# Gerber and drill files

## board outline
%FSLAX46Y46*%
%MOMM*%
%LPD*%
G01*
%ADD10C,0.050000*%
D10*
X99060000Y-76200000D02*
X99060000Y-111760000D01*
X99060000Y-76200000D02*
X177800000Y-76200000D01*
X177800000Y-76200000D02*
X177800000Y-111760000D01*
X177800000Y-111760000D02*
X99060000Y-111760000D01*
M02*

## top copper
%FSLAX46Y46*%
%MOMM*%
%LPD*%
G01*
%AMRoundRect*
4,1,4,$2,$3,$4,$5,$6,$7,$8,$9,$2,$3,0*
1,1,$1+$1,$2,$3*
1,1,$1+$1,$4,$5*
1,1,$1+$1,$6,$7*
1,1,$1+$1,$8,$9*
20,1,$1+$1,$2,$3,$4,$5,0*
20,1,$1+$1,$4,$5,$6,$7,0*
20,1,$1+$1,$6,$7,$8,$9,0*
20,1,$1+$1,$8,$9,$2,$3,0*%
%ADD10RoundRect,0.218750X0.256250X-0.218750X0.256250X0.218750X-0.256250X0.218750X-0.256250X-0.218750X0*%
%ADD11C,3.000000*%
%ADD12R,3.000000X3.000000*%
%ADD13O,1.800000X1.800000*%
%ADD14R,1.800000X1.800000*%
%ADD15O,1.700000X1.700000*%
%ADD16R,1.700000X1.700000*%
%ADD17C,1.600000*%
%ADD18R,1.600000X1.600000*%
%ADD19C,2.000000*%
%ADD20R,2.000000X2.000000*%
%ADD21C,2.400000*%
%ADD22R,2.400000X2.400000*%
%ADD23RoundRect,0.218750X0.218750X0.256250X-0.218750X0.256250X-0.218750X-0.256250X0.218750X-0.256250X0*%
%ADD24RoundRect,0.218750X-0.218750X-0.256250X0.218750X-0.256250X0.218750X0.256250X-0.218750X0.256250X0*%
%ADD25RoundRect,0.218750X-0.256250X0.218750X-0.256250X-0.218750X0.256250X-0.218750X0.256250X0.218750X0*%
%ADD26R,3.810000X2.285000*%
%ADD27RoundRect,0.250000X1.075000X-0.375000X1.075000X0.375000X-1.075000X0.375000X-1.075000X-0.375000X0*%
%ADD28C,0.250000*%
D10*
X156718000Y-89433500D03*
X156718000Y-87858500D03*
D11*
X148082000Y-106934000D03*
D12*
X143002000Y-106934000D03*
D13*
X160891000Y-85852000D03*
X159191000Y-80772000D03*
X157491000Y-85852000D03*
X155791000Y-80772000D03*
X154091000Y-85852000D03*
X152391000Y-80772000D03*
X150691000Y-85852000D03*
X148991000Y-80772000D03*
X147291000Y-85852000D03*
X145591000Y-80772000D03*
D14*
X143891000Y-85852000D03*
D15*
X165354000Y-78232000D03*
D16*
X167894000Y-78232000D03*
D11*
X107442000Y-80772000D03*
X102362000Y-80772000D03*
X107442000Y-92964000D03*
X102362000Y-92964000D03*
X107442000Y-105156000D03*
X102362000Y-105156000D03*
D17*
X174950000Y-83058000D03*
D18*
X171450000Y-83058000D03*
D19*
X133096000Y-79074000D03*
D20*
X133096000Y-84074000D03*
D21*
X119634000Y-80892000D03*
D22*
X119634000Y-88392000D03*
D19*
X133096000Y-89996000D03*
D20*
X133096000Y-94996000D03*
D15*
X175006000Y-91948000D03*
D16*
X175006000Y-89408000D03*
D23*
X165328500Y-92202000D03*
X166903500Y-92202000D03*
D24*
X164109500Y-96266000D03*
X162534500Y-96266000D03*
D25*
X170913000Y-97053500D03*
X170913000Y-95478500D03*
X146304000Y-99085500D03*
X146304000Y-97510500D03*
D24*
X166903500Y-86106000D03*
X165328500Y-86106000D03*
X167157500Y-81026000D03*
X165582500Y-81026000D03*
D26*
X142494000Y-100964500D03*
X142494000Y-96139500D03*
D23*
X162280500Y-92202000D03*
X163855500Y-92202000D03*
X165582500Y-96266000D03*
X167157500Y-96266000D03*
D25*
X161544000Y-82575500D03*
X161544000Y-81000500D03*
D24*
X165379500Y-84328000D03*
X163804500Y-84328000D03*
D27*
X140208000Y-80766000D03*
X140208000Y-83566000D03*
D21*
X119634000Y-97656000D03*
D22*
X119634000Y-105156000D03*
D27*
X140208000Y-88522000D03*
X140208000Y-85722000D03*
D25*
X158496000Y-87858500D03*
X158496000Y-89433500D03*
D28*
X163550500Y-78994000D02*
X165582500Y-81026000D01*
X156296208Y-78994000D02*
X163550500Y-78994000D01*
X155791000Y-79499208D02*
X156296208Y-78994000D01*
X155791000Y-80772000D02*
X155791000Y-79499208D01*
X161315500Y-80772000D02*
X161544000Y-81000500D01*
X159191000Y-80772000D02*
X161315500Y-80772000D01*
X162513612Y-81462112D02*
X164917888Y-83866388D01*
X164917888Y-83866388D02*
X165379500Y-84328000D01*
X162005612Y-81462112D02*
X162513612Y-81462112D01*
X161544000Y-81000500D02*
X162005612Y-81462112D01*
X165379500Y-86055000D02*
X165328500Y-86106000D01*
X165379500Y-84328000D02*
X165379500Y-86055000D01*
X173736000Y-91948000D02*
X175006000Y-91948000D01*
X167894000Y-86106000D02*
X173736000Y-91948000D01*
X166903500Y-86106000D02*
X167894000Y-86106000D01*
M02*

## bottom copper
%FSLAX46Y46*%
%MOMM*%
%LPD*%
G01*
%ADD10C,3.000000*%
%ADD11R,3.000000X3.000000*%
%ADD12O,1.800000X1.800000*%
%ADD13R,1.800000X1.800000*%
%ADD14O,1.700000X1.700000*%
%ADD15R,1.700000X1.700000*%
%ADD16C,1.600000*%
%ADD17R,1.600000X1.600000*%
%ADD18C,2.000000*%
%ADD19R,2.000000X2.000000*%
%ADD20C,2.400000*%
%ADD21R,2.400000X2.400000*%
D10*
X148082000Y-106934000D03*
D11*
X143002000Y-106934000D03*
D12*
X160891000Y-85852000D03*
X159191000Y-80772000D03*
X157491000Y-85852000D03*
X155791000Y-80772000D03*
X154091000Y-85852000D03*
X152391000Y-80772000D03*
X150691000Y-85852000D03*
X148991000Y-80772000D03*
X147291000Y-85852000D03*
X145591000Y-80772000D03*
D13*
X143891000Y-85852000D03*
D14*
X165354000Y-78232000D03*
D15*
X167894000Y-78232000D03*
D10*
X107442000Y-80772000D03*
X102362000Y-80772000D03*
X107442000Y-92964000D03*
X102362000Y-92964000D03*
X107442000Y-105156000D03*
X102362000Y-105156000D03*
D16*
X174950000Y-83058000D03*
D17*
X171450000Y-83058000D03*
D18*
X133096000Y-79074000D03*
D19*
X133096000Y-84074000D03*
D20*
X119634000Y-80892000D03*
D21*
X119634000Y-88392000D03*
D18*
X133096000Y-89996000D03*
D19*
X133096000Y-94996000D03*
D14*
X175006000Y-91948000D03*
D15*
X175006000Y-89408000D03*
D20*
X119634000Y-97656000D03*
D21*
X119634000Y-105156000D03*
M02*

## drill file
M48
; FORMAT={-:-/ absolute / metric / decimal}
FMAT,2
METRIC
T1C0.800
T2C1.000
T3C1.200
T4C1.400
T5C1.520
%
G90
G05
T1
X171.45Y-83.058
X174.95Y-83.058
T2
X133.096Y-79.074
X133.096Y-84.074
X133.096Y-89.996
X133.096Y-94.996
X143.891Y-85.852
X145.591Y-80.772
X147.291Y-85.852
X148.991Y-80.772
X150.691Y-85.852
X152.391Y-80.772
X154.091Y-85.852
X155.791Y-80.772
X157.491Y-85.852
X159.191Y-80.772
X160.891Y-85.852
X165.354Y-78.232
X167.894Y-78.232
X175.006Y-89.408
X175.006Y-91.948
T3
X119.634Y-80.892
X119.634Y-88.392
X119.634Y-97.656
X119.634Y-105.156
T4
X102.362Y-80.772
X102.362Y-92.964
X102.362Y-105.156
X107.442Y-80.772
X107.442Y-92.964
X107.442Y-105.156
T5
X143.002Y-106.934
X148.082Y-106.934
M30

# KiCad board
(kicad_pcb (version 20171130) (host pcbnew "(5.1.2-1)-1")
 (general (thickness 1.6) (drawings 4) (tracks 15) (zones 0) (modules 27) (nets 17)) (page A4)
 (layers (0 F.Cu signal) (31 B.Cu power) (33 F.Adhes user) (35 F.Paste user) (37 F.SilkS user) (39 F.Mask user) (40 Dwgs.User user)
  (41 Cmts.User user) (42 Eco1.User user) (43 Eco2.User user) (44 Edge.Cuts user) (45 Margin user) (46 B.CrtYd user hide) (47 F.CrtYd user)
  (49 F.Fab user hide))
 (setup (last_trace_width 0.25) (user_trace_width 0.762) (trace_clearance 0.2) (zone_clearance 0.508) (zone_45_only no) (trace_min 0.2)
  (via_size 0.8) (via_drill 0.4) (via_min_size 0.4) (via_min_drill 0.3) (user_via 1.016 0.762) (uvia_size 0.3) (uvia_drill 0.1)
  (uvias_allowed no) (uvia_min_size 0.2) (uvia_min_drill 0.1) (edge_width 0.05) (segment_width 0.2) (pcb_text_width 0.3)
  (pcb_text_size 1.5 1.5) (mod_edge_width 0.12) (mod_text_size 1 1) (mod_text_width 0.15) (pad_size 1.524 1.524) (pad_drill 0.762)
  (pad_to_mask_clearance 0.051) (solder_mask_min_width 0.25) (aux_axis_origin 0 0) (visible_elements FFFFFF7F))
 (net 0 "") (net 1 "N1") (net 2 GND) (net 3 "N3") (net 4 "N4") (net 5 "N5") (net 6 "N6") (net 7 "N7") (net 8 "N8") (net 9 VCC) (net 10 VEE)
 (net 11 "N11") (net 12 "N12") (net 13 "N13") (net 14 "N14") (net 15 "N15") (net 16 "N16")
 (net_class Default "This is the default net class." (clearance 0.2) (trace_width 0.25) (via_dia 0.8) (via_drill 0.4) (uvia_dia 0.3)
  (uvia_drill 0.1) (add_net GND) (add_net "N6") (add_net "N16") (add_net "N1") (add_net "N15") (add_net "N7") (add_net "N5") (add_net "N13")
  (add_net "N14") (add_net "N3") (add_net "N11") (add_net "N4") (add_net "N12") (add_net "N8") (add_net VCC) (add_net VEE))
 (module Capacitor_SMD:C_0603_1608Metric (layer F.Cu) (at 156.718 88.646 90)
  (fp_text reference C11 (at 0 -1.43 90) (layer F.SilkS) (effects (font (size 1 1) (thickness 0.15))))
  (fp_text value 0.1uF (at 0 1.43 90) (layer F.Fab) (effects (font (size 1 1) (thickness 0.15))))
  (pad 1 smd roundrect (at -0.7875 0 90) (size 0.875 0.95) (layers F.Cu F.Paste F.Mask) (roundrect_rratio 0.25) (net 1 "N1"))
  (pad 2 smd roundrect (at 0.7875 0 90) (size 0.875 0.95) (layers F.Cu F.Paste F.Mask) (roundrect_rratio 0.25) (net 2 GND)))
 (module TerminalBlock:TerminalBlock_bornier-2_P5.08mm (layer F.Cu) (at 143.002 106.934)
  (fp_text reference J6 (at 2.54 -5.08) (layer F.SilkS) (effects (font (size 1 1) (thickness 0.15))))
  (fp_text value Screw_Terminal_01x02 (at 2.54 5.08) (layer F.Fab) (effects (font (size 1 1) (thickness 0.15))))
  (pad 2 thru_hole circle (at 5.08 0) (size 3 3) (drill 1.52) (layers *.Cu *.Mask) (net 2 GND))
  (pad 1 thru_hole rect (at 0 0) (size 3 3) (drill 1.52) (layers *.Cu *.Mask) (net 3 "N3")))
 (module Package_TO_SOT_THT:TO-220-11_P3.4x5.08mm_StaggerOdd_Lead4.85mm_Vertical (layer F.Cu) (at 143.891 85.852)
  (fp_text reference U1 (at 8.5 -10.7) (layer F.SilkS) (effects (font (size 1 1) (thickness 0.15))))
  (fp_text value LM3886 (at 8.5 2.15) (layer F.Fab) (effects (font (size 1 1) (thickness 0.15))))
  (pad 11 thru_hole oval (at 17 0) (size 1.8 1.8) (drill 1) (layers *.Cu *.Mask) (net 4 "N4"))
  (pad 10 thru_hole oval (at 15.3 -5.08) (size 1.8 1.8) (drill 1) (layers *.Cu *.Mask) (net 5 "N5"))
  (pad 9 thru_hole oval (at 13.6 0) (size 1.8 1.8) (drill 1) (layers *.Cu *.Mask) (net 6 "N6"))
  (pad 8 thru_hole oval (at 11.9 -5.08) (size 1.8 1.8) (drill 1) (layers *.Cu *.Mask) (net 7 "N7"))
  (pad 7 thru_hole oval (at 10.2 0) (size 1.8 1.8) (drill 1) (layers *.Cu *.Mask) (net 2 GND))
  (pad 6 thru_hole oval (at 8.5 -5.08) (size 1.8 1.8) (drill 1) (layers *.Cu *.Mask) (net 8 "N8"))
  (pad 5 thru_hole oval (at 6.8 0) (size 1.8 1.8) (drill 1) (layers *.Cu *.Mask) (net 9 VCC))
  (pad 4 thru_hole oval (at 5.1 -5.08) (size 1.8 1.8) (drill 1) (layers *.Cu *.Mask) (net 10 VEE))
  (pad 3 thru_hole oval (at 3.4 0) (size 1.8 1.8) (drill 1) (layers *.Cu *.Mask) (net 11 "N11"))
  (pad 2 thru_hole oval (at 1.7 -5.08) (size 1.8 1.8) (drill 1) (layers *.Cu *.Mask) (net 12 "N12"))
  (pad 1 thru_hole rect (at 0 0) (size 1.8 1.8) (drill 1) (layers *.Cu *.Mask) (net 9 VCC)))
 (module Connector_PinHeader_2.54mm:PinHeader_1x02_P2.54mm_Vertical (layer F.Cu) (at 167.894 78.232 270)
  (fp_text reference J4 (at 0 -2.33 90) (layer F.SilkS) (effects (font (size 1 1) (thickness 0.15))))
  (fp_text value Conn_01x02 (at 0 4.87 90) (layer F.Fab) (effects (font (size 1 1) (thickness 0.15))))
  (pad 2 thru_hole oval (at 0 2.54 270) (size 1.7 1.7) (drill 1) (layers *.Cu *.Mask) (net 10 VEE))
  (pad 1 thru_hole rect (at 0 0 270) (size 1.7 1.7) (drill 1) (layers *.Cu *.Mask) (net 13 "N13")))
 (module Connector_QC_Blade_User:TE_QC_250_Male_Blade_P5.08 (layer F.Cu) (at 107.442 80.772 180)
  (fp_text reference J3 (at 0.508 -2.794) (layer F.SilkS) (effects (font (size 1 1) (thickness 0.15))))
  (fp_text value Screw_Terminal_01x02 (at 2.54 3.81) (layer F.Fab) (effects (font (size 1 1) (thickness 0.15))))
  (pad 1 thru_hole circle (at 0 0 180) (size 3 3) (drill 1.4) (layers *.Cu *.Mask) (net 10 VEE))
  (pad 2 thru_hole circle (at 5.08 0 180) (size 3 3) (drill 1.4) (layers *.Cu *.Mask) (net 10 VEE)))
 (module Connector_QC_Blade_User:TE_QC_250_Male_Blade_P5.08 (layer F.Cu) (at 107.442 92.964 180)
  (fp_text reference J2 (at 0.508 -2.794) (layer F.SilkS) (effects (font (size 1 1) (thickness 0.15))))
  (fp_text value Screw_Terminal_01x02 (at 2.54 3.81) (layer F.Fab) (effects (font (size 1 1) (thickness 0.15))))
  (pad 1 thru_hole circle (at 0 0 180) (size 3 3) (drill 1.4) (layers *.Cu *.Mask) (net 2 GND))
  (pad 2 thru_hole circle (at 5.08 0 180) (size 3 3) (drill 1.4) (layers *.Cu *.Mask) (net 2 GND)))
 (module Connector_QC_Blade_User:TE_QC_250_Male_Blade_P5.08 (layer F.Cu) (at 107.442 105.156 180)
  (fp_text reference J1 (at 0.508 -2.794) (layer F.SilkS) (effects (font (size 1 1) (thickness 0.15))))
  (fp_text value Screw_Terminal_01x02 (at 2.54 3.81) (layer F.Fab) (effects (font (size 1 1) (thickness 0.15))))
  (pad 1 thru_hole circle (at 0 0 180) (size 3 3) (drill 1.4) (layers *.Cu *.Mask) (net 9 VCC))
  (pad 2 thru_hole circle (at 5.08 0 180) (size 3 3) (drill 1.4) (layers *.Cu *.Mask) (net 9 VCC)))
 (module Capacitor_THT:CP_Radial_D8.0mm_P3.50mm (layer F.Cu) (at 171.45 83.058)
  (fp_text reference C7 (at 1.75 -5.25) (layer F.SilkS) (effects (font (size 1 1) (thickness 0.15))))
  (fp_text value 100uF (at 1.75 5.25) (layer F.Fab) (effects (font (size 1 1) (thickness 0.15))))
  (pad 2 thru_hole circle (at 3.5 0) (size 1.6 1.6) (drill 0.8) (layers *.Cu *.Mask) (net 2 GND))
  (pad 1 thru_hole rect (at 0 0) (size 1.6 1.6) (drill 0.8) (layers *.Cu *.Mask) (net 7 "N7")))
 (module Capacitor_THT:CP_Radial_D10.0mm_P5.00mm (layer F.Cu) (at 133.096 84.074 90)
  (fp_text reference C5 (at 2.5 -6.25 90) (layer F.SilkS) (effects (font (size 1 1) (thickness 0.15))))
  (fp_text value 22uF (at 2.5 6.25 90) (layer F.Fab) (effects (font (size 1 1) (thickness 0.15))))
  (pad 2 thru_hole circle (at 5 0 90) (size 2 2) (drill 1) (layers *.Cu *.Mask) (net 10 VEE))
  (pad 1 thru_hole rect (at 0 0 90) (size 2 2) (drill 1) (layers *.Cu *.Mask) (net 2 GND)))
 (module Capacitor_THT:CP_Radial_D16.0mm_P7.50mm (layer F.Cu) (at 119.634 88.392 90)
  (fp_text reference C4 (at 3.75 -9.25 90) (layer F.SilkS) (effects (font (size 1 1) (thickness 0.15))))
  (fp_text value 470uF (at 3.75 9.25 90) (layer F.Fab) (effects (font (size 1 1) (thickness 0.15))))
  (pad 2 thru_hole circle (at 7.5 0 90) (size 2.4 2.4) (drill 1.2) (layers *.Cu *.Mask) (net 10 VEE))
  (pad 1 thru_hole rect (at 0 0 90) (size 2.4 2.4) (drill 1.2) (layers *.Cu *.Mask) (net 2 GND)))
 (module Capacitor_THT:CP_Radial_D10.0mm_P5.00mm (layer F.Cu) (at 133.096 94.996 90)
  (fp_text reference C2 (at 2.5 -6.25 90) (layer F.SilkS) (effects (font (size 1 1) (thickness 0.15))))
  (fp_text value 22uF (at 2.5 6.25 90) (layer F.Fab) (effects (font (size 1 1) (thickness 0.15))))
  (pad 2 thru_hole circle (at 5 0 90) (size 2 2) (drill 1) (layers *.Cu *.Mask) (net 2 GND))
  (pad 1 thru_hole rect (at 0 0 90) (size 2 2) (drill 1) (layers *.Cu *.Mask) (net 9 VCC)))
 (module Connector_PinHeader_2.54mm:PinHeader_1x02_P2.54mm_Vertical (layer F.Cu) (at 175.006 89.408)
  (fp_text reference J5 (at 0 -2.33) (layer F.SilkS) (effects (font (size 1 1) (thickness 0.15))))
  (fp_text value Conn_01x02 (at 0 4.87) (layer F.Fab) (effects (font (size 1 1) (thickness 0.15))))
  (pad 2 thru_hole oval (at 0 2.54) (size 1.7 1.7) (drill 1) (layers *.Cu *.Mask) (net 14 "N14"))
  (pad 1 thru_hole rect (at 0 0) (size 1.7 1.7) (drill 1) (layers *.Cu *.Mask) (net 2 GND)))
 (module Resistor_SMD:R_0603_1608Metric (layer F.Cu) (at 166.116 92.202 180)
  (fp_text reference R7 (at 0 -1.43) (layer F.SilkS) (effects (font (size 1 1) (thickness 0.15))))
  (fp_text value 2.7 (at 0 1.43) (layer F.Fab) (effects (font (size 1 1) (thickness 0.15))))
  (pad 2 smd roundrect (at 0.7875 0 180) (size 0.875 0.95) (layers F.Cu F.Paste F.Mask) (roundrect_rratio 0.25) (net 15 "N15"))
  (pad 1 smd roundrect (at -0.7875 0 180) (size 0.875 0.95) (layers F.Cu F.Paste F.Mask) (roundrect_rratio 0.25) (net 11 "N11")))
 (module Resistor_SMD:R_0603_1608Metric (layer F.Cu) (at 163.322 96.266)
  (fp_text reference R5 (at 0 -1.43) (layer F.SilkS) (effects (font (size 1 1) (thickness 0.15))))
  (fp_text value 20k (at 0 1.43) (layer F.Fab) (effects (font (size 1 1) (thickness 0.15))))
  (pad 2 smd roundrect (at 0.7875 0) (size 0.875 0.95) (layers F.Cu F.Paste F.Mask) (roundrect_rratio 0.25) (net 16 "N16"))
  (pad 1 smd roundrect (at -0.7875 0) (size 0.875 0.95) (layers F.Cu F.Paste F.Mask) (roundrect_rratio 0.25) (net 11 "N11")))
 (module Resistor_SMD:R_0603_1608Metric (layer F.Cu) (at 170.913 96.266 270)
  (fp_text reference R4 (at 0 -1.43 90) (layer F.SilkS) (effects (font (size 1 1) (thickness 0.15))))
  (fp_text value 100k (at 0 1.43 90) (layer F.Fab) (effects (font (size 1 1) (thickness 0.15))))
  (pad 2 smd roundrect (at 0.7875 0 270) (size 0.875 0.95) (layers F.Cu F.Paste F.Mask) (roundrect_rratio 0.25) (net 6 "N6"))
  (pad 1 smd roundrect (at -0.7875 0 270) (size 0.875 0.95) (layers F.Cu F.Paste F.Mask) (roundrect_rratio 0.25) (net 11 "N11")))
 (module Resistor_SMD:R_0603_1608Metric (layer F.Cu) (at 146.304 98.298 270)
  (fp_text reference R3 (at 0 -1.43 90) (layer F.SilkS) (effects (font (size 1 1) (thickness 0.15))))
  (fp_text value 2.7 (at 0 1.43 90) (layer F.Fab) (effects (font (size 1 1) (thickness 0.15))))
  (pad 2 smd roundrect (at 0.7875 0 270) (size 0.875 0.95) (layers F.Cu F.Paste F.Mask) (roundrect_rratio 0.25) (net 3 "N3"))
  (pad 1 smd roundrect (at -0.7875 0 270) (size 0.875 0.95) (layers F.Cu F.Paste F.Mask) (roundrect_rratio 0.25) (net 11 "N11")))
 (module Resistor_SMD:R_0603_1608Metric (layer F.Cu) (at 166.116 86.106)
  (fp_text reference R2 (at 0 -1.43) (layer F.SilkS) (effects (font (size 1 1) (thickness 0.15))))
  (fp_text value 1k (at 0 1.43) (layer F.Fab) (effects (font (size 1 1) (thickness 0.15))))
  (pad 2 smd roundrect (at 0.7875 0) (size 0.875 0.95) (layers F.Cu F.Paste F.Mask) (roundrect_rratio 0.25) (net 14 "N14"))
  (pad 1 smd roundrect (at -0.7875 0) (size 0.875 0.95) (layers F.Cu F.Paste F.Mask) (roundrect_rratio 0.25) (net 5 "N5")))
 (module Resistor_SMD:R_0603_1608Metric (layer F.Cu) (at 166.37 81.026)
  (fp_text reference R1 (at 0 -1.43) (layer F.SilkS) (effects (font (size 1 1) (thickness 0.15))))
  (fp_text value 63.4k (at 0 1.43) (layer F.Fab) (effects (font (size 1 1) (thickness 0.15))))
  (pad 2 smd roundrect (at 0.7875 0) (size 0.875 0.95) (layers F.Cu F.Paste F.Mask) (roundrect_rratio 0.25) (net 13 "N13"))
  (pad 1 smd roundrect (at -0.7875 0) (size 0.875 0.95) (layers F.Cu F.Paste F.Mask) (roundrect_rratio 0.25) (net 7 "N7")))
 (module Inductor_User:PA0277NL (layer F.Cu) (at 142.494 98.552 270)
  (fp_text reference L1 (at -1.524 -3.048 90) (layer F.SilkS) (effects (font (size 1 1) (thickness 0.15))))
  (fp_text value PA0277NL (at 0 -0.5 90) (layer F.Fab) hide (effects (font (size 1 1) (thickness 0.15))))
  (pad 2 smd rect (at 2.4125 0 270) (size 2.285 3.81) (layers F.Cu F.Paste F.Mask) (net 3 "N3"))
  (pad 1 smd rect (at -2.4125 0 270) (size 2.285 3.81) (layers F.Cu F.Paste F.Mask) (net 11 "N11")))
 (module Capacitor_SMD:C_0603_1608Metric (layer F.Cu) (at 163.068 92.202 180)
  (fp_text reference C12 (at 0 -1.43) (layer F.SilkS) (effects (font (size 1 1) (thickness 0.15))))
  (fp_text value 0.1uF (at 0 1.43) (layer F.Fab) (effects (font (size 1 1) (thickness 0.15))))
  (pad 2 smd roundrect (at 0.7875 0 180) (size 0.875 0.95) (layers F.Cu F.Paste F.Mask) (roundrect_rratio 0.25) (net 2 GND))
  (pad 1 smd roundrect (at -0.7875 0 180) (size 0.875 0.95) (layers F.Cu F.Paste F.Mask) (roundrect_rratio 0.25) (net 15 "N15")))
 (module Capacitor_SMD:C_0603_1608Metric (layer F.Cu) (at 166.37 96.266 180)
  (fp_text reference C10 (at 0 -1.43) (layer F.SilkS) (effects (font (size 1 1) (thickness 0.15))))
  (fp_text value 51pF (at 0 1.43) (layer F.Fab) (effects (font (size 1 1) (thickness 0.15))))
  (pad 2 smd roundrect (at 0.7875 0 180) (size 0.875 0.95) (layers F.Cu F.Paste F.Mask) (roundrect_rratio 0.25) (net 16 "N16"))
  (pad 1 smd roundrect (at -0.7875 0 180) (size 0.875 0.95) (layers F.Cu F.Paste F.Mask) (roundrect_rratio 0.25) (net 6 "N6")))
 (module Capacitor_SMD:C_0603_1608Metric (layer F.Cu) (at 161.544 81.788 270)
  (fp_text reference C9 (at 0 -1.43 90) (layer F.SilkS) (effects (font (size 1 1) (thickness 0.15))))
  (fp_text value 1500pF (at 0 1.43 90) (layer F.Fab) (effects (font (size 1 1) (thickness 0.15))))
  (pad 2 smd roundrect (at 0.7875 0 270) (size 0.875 0.95) (layers F.Cu F.Paste F.Mask) (roundrect_rratio 0.25) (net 2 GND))
  (pad 1 smd roundrect (at -0.7875 0 270) (size 0.875 0.95) (layers F.Cu F.Paste F.Mask) (roundrect_rratio 0.25) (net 5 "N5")))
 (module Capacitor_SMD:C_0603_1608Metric (layer F.Cu) (at 164.592 84.328)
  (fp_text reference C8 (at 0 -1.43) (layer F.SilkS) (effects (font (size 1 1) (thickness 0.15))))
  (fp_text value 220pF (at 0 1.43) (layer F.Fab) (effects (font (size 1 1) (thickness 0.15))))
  (pad 2 smd roundrect (at 0.7875 0) (size 0.875 0.95) (layers F.Cu F.Paste F.Mask) (roundrect_rratio 0.25) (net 5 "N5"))
  (pad 1 smd roundrect (at -0.7875 0) (size 0.875 0.95) (layers F.Cu F.Paste F.Mask) (roundrect_rratio 0.25) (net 6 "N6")))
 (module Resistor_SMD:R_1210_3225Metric (layer F.Cu) (at 140.208 82.166 90)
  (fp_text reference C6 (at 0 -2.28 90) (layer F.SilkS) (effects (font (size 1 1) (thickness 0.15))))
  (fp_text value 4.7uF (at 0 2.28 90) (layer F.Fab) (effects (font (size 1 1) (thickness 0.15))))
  (pad 2 smd roundrect (at 1.4 0 90) (size 1.25 2.65) (layers F.Cu F.Paste F.Mask) (roundrect_rratio 0.2) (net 10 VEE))
  (pad 1 smd roundrect (at -1.4 0 90) (size 1.25 2.65) (layers F.Cu F.Paste F.Mask) (roundrect_rratio 0.2) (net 2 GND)))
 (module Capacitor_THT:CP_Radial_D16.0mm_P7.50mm (layer F.Cu) (at 119.634 105.156 90)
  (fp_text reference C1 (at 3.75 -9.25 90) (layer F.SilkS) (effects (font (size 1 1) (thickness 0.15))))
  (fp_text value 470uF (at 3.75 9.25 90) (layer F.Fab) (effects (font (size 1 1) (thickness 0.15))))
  (pad 2 thru_hole circle (at 7.5 0 90) (size 2.4 2.4) (drill 1.2) (layers *.Cu *.Mask) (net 2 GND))
  (pad 1 thru_hole rect (at 0 0 90) (size 2.4 2.4) (drill 1.2) (layers *.Cu *.Mask) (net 9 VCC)))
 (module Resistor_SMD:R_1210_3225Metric (layer F.Cu) (at 140.208 87.122 90)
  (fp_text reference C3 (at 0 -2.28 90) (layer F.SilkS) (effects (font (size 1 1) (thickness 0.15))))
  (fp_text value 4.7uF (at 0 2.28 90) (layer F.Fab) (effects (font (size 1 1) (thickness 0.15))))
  (pad 1 smd roundrect (at -1.4 0 90) (size 1.25 2.65) (layers F.Cu F.Paste F.Mask) (roundrect_rratio 0.2) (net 9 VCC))
  (pad 2 smd roundrect (at 1.4 0 90) (size 1.25 2.65) (layers F.Cu F.Paste F.Mask) (roundrect_rratio 0.2) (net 2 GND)))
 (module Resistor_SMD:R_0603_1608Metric (layer F.Cu) (at 158.496 88.646 270)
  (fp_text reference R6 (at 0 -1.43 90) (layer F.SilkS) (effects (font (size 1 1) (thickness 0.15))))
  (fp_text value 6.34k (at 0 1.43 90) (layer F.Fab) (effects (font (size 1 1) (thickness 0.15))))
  (pad 1 smd roundrect (at -0.7875 0 270) (size 0.875 0.95) (layers F.Cu F.Paste F.Mask) (roundrect_rratio 0.25) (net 6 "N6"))
  (pad 2 smd roundrect (at 0.7875 0 270) (size 0.875 0.95) (layers F.Cu F.Paste F.Mask) (roundrect_rratio 0.25) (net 1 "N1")))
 (gr_line (start 99.06 76.2) (end 99.06 111.76) (layer Edge.Cuts) (width 0.05))
 (gr_line (start 99.06 76.2) (end 177.8 76.2) (layer Edge.Cuts) (width 0.05))
 (gr_line (start 177.8 76.2) (end 177.8 111.76) (layer Edge.Cuts) (width 0.05))
 (gr_line (start 177.8 111.76) (end 99.06 111.76) (layer Edge.Cuts) (width 0.05))
 (segment (start 163.5505 78.994) (end 165.5825 81.026) (width 0.25) (layer F.Cu) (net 7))
 (segment (start 156.296208 78.994) (end 163.5505 78.994) (width 0.25) (layer F.Cu) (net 7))
 (segment (start 155.791 79.499208) (end 156.296208 78.994) (width 0.25) (layer F.Cu) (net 7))
 (segment (start 155.791 80.772) (end 155.791 79.499208) (width 0.25) (layer F.Cu) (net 7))
 (segment (start 161.3155 80.772) (end 161.544 81.0005) (width 0.25) (layer F.Cu) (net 5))
 (segment (start 159.191 80.772) (end 161.3155 80.772) (width 0.25) (layer F.Cu) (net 5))
 (segment (start 162.513612 81.462112) (end 164.917888 83.866388) (width 0.25) (layer F.Cu) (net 5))
 (segment (start 164.917888 83.866388) (end 165.3795 84.328) (width 0.25) (layer F.Cu) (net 5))
 (segment (start 162.005612 81.462112) (end 162.513612 81.462112) (width 0.25) (layer F.Cu) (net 5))
 (segment (start 161.544 81.0005) (end 162.005612 81.462112) (width 0.25) (layer F.Cu) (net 5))
 (segment (start 165.3795 86.055) (end 165.3285 86.106) (width 0.25) (layer F.Cu) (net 5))
 (segment (start 165.3795 84.328) (end 165.3795 86.055) (width 0.25) (layer F.Cu) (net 5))
 (segment (start 173.736 91.948) (end 175.006 91.948) (width 0.25) (layer F.Cu) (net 14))
 (segment (start 167.894 86.106) (end 173.736 91.948) (width 0.25) (layer F.Cu) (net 14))
 (segment (start 166.9035 86.106) (end 167.894 86.106) (width 0.25) (layer F.Cu) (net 14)))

